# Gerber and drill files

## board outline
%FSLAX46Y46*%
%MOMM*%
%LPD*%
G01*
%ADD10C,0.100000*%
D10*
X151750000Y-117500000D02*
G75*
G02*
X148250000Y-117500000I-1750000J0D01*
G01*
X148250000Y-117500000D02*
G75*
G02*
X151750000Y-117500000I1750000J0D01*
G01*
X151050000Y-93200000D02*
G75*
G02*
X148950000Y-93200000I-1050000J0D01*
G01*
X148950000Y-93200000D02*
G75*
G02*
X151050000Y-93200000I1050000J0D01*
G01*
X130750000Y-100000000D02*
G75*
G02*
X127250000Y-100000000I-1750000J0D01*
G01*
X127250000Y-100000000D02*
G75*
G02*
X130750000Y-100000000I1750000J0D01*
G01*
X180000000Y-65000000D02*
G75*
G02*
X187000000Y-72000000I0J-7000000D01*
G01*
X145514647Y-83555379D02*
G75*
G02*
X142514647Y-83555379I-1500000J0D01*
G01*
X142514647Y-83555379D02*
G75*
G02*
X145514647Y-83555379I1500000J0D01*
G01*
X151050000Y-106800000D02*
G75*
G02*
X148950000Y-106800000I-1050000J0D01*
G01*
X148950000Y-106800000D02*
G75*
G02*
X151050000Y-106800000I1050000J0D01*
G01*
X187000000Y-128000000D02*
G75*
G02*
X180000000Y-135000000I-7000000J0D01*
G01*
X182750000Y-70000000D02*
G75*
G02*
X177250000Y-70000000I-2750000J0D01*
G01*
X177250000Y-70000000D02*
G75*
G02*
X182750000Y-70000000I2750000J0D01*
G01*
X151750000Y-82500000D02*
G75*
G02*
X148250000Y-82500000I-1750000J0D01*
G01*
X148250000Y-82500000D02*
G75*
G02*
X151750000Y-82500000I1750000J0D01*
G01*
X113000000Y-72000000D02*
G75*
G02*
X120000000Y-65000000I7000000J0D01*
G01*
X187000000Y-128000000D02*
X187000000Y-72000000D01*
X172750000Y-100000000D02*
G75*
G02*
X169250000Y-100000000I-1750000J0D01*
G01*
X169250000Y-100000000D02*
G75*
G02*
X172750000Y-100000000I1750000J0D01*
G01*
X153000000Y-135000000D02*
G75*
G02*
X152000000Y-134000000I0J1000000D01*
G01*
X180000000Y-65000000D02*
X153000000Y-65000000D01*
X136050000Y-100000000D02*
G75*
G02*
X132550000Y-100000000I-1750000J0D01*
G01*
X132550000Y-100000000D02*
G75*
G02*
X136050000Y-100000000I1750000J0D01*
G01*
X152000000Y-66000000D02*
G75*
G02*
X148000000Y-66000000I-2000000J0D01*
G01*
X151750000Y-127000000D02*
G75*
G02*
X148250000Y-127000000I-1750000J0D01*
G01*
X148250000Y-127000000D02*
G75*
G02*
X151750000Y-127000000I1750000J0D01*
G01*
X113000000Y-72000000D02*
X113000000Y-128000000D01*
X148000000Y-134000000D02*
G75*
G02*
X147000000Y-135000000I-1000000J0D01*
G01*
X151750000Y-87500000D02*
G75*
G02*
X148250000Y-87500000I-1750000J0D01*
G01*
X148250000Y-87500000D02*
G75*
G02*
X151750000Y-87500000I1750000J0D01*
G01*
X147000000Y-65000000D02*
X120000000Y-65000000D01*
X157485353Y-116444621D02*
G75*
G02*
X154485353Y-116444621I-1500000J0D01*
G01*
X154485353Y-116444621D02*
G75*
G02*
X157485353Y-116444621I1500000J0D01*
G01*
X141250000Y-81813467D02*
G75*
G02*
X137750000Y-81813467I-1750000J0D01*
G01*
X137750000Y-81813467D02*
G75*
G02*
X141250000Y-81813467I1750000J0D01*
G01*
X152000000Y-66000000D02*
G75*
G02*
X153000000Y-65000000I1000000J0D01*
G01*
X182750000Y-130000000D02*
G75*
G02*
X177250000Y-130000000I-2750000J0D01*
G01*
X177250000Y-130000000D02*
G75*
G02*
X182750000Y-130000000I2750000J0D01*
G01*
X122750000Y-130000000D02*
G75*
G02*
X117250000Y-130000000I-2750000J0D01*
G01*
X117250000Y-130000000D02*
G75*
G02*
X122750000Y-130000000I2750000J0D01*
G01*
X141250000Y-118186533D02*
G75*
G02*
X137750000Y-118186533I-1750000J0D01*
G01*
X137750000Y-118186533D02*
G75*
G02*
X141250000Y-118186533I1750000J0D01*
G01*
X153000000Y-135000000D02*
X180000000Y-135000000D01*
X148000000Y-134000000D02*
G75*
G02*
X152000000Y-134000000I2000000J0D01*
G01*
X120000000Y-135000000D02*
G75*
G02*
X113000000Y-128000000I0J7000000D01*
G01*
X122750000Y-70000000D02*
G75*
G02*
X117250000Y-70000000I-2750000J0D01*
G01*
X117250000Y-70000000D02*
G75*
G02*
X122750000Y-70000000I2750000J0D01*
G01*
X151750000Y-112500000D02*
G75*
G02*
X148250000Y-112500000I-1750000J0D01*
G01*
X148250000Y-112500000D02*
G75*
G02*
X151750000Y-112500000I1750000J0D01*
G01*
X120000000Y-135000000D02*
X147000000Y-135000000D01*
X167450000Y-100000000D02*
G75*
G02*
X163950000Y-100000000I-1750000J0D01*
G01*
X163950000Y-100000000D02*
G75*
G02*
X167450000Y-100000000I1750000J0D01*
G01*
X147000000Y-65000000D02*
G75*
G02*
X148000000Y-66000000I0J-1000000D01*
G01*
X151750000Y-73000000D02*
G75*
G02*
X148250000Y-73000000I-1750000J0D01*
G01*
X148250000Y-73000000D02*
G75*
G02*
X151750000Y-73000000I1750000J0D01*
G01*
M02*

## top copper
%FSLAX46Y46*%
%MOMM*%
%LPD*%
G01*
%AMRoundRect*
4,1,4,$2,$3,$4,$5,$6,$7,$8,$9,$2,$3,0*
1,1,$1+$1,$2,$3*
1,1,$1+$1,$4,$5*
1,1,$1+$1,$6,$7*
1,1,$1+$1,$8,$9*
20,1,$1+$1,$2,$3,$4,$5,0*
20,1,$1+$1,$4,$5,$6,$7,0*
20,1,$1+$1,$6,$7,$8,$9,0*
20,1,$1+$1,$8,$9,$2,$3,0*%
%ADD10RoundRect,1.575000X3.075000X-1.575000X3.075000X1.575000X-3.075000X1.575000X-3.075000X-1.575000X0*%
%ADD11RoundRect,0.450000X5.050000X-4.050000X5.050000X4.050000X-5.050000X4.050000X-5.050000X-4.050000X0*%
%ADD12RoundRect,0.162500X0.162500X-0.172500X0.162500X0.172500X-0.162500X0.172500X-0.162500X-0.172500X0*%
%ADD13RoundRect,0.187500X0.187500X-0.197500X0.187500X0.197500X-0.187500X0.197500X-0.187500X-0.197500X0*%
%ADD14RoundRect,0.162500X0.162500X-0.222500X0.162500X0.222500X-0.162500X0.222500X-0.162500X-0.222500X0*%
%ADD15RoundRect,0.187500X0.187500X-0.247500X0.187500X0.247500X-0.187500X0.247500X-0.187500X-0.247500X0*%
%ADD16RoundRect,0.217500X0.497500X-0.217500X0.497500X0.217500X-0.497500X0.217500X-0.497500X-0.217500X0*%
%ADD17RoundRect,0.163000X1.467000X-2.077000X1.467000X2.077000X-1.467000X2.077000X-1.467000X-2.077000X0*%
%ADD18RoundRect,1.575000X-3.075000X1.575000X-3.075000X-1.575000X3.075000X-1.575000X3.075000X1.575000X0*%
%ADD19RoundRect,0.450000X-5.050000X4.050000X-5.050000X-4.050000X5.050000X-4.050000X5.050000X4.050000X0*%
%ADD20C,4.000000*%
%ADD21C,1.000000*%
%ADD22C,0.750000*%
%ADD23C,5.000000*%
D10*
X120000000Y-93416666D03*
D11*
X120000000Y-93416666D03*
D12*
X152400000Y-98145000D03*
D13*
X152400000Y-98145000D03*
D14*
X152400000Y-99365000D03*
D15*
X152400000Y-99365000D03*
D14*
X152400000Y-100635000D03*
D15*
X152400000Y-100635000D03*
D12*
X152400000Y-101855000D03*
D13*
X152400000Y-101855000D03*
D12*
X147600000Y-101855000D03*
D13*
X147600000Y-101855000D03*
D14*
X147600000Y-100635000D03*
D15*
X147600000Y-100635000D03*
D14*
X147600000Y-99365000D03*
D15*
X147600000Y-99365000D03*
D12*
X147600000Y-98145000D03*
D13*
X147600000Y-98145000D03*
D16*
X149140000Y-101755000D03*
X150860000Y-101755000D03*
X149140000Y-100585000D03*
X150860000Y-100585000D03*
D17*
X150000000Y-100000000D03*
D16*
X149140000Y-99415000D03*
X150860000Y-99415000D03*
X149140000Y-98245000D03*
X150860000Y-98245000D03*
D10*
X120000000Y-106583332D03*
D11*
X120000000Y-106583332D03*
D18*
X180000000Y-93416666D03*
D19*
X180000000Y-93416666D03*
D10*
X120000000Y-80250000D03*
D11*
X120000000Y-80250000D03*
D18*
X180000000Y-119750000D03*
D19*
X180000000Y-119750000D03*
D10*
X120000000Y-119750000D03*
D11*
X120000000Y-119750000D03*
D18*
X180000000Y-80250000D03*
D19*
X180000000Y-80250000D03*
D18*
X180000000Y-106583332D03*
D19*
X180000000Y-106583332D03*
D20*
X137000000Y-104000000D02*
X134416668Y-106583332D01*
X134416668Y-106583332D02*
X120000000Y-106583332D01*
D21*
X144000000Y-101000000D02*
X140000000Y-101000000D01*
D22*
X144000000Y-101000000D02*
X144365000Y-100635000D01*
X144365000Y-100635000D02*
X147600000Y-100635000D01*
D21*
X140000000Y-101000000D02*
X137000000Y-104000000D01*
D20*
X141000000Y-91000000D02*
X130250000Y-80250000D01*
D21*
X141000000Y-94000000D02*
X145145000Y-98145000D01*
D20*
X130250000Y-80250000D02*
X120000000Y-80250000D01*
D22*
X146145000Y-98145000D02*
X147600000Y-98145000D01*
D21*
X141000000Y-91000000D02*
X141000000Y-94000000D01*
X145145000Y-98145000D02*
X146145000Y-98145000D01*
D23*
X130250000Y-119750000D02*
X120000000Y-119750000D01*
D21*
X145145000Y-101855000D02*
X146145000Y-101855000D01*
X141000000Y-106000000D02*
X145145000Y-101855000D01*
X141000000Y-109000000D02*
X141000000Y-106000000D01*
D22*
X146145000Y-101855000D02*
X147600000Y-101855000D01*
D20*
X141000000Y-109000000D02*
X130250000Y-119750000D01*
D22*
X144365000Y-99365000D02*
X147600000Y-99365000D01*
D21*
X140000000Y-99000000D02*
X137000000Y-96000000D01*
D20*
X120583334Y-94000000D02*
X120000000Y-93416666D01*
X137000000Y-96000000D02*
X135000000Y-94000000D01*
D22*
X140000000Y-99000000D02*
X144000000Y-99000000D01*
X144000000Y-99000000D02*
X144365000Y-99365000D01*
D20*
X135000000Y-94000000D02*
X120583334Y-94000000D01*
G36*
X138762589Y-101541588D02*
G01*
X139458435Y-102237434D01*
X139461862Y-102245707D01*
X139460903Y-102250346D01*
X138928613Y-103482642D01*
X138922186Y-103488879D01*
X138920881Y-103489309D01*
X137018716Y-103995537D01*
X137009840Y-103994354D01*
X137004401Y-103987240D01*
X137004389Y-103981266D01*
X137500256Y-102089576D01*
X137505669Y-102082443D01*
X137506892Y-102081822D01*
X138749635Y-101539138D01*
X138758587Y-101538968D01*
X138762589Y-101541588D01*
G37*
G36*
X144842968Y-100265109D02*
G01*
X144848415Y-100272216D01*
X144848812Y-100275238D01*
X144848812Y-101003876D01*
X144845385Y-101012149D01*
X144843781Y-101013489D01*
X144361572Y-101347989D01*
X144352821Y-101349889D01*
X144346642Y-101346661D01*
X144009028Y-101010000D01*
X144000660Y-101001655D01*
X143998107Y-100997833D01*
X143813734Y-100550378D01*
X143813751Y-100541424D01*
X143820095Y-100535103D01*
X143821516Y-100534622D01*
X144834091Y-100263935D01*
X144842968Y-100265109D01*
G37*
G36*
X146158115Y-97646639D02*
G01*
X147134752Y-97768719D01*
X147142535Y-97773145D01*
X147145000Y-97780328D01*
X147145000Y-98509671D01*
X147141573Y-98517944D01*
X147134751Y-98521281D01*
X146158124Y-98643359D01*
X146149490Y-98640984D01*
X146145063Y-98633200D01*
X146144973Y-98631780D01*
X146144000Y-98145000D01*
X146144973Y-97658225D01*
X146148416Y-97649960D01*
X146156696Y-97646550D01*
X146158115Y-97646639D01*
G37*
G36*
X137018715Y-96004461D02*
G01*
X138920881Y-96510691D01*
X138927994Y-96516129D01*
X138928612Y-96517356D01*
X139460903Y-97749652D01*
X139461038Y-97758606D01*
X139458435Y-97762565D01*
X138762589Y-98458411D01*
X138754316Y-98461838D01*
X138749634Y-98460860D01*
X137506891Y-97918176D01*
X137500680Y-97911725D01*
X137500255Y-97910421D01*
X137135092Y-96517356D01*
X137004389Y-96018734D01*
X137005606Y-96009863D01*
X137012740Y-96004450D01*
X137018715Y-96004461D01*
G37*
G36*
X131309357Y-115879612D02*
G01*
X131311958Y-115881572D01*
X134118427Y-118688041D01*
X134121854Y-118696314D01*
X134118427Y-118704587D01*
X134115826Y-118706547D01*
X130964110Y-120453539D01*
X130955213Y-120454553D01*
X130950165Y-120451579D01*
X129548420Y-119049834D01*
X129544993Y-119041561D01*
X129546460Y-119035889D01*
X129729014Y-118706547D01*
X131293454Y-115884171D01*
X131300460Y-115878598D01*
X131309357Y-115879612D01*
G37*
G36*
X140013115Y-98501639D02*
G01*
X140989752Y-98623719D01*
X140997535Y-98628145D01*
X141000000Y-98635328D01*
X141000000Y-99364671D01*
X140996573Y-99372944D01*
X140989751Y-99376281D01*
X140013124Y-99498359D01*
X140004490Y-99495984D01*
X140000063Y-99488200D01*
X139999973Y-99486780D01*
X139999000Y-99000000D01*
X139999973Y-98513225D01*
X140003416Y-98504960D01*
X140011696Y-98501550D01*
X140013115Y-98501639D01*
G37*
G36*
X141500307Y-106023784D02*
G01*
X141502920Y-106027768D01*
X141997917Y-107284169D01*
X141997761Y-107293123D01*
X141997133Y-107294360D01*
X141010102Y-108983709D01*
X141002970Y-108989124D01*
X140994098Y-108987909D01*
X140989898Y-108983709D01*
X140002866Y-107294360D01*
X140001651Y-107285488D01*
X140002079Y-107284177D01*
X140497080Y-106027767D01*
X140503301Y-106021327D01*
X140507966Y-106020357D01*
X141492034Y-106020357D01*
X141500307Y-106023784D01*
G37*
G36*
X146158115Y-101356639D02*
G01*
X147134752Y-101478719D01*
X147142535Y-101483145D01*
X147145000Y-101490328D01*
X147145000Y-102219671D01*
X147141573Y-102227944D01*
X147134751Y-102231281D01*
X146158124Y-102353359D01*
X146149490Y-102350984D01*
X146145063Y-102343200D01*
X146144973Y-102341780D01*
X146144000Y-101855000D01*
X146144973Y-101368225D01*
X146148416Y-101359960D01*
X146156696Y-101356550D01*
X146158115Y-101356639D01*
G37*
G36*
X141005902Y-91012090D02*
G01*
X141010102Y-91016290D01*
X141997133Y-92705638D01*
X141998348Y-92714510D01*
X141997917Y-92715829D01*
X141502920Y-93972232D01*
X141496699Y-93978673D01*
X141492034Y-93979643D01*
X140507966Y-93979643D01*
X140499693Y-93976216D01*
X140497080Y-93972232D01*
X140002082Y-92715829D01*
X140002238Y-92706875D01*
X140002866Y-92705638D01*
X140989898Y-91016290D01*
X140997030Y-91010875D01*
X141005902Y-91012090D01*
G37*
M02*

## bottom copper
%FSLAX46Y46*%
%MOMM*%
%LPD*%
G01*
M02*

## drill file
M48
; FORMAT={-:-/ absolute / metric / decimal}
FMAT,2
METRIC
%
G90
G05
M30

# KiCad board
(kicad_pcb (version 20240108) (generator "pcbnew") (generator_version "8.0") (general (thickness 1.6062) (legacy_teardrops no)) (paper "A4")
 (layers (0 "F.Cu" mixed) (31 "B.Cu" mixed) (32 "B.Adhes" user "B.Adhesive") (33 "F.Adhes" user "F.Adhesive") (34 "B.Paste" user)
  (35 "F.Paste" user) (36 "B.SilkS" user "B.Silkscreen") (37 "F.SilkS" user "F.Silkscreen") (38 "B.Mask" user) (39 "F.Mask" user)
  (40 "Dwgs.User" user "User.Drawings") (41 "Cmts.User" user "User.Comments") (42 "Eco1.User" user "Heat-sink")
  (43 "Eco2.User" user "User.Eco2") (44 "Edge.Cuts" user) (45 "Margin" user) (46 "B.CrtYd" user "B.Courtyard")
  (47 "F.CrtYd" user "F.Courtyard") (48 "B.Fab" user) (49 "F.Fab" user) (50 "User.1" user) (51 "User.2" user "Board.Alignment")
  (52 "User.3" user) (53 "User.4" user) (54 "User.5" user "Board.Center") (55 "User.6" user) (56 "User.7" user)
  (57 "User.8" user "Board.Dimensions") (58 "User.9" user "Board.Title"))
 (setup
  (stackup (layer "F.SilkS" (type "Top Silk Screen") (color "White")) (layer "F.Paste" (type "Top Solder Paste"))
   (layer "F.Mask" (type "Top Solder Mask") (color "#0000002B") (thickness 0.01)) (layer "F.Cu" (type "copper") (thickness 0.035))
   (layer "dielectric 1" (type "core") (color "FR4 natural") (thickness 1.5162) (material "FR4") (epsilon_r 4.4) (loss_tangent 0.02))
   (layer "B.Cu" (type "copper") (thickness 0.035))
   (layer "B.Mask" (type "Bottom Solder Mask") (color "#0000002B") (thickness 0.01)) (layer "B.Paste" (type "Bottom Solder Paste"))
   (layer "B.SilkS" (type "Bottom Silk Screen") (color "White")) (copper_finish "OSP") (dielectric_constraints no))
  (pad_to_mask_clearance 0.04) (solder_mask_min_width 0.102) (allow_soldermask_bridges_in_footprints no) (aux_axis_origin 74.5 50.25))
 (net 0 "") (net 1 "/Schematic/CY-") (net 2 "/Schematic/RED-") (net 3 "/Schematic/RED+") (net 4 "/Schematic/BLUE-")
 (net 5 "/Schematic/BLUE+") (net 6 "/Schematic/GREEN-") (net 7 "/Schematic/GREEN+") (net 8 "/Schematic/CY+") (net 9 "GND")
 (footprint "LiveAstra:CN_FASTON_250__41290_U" (layer "F.Cu") (at 120 93.416666 90)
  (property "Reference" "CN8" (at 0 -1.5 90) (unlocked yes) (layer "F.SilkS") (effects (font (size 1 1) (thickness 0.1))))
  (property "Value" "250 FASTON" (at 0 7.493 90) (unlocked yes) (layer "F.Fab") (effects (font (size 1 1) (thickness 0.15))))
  (pad "1" smd roundrect (at 0 0 90) (size 6.3 9.3) (layers "F.Cu" "F.Paste") (roundrect_rratio 0.25) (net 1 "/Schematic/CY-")
   (thermal_bridge_angle 45)
   (teardrops (best_length_ratio 0.5) (max_length 1) (best_width_ratio 1) (max_width 2) (curve_points 0) (filter_ratio 0.9) (enabled yes)
    (allow_two_segments yes) (prefer_zone_connections yes)))
  (pad "1" smd roundrect (at 0 0 90) (size 9 11) (layers "F.Cu" "F.Mask") (roundrect_rratio 0.05) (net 1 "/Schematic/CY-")
   (thermal_bridge_angle 45)
   (teardrops (best_length_ratio 0.5) (max_length 1) (best_width_ratio 1) (max_width 2) (curve_points 0) (filter_ratio 0.9) (enabled yes)
    (allow_two_segments yes) (prefer_zone_connections yes))))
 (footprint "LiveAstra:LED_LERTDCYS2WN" (layer "F.Cu") (at 150 100 90)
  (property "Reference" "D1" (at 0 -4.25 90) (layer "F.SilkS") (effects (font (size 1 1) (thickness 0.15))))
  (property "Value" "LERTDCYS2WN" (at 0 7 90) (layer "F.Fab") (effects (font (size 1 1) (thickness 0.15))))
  (pad "1" smd roundrect (at 1.855 2.4 90) (size 0.67 0.65) (layers "F.Cu" "F.Paste") (roundrect_rratio 0.25) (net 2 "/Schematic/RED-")
   (thermal_bridge_angle 45)
   (teardrops (best_length_ratio 0.5) (max_length 1) (best_width_ratio 1) (max_width 2) (curve_points 0) (filter_ratio 0.9) (enabled yes)
    (allow_two_segments yes) (prefer_zone_connections yes)))
  (pad "1" smd roundrect (at 1.855 2.4 90) (size 0.77 0.75) (layers "F.Cu" "F.Mask") (roundrect_rratio 0.25) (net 2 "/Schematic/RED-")
   (thermal_bridge_angle 45)
   (teardrops (best_length_ratio 0.5) (max_length 1) (best_width_ratio 1) (max_width 2) (curve_points 0) (filter_ratio 0.9) (enabled yes)
    (allow_two_segments yes) (prefer_zone_connections yes)))
  (pad "2" smd roundrect (at 0.635 2.4 90) (size 0.77 0.65) (layers "F.Cu" "F.Paste") (roundrect_rratio 0.25) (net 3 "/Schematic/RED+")
   (thermal_bridge_angle 45)
   (teardrops (best_length_ratio 0.5) (max_length 1) (best_width_ratio 1) (max_width 2) (curve_points 0) (filter_ratio 0.9) (enabled yes)
    (allow_two_segments yes) (prefer_zone_connections yes)))
  (pad "2" smd roundrect (at 0.635 2.4 90) (size 0.87 0.75) (layers "F.Cu" "F.Mask") (roundrect_rratio 0.25) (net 3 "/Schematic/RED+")
   (thermal_bridge_angle 45)
   (teardrops (best_length_ratio 0.5) (max_length 1) (best_width_ratio 1) (max_width 2) (curve_points 0) (filter_ratio 0.9) (enabled yes)
    (allow_two_segments yes) (prefer_zone_connections yes)))
  (pad "3" smd roundrect (at -0.635 2.4 90) (size 0.77 0.65) (layers "F.Cu" "F.Paste") (roundrect_rratio 0.25) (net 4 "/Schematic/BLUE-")
   (thermal_bridge_angle 45)
   (teardrops (best_length_ratio 0.5) (max_length 1) (best_width_ratio 1) (max_width 2) (curve_points 0) (filter_ratio 0.9) (enabled yes)
    (allow_two_segments yes) (prefer_zone_connections yes)))
  (pad "3" smd roundrect (at -0.635 2.4 90) (size 0.87 0.75) (layers "F.Cu" "F.Mask") (roundrect_rratio 0.25) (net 4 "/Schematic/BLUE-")
   (thermal_bridge_angle 45)
   (teardrops (best_length_ratio 0.5) (max_length 1) (best_width_ratio 1) (max_width 2) (curve_points 0) (filter_ratio 0.9) (enabled yes)
    (allow_two_segments yes) (prefer_zone_connections yes)))
  (pad "4" smd roundrect (at -1.855 2.4 90) (size 0.67 0.65) (layers "F.Cu" "F.Paste") (roundrect_rratio 0.25) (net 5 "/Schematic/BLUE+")
   (thermal_bridge_angle 45)
   (teardrops (best_length_ratio 0.5) (max_length 1) (best_width_ratio 1) (max_width 2) (curve_points 0) (filter_ratio 0.9) (enabled yes)
    (allow_two_segments yes) (prefer_zone_connections yes)))
  (pad "4" smd roundrect (at -1.855 2.4 90) (size 0.77 0.75) (layers "F.Cu" "F.Mask") (roundrect_rratio 0.25) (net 5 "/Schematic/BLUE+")
   (thermal_bridge_angle 45)
   (teardrops (best_length_ratio 0.5) (max_length 1) (best_width_ratio 1) (max_width 2) (curve_points 0) (filter_ratio 0.9) (enabled yes)
    (allow_two_segments yes) (prefer_zone_connections yes)))
  (pad "5" smd roundrect (at -1.855 -2.4 90) (size 0.67 0.65) (layers "F.Cu" "F.Paste") (roundrect_rratio 0.25) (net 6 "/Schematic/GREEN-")
   (thermal_bridge_angle 45)
   (teardrops (best_length_ratio 0.5) (max_length 1) (best_width_ratio 1) (max_width 2) (curve_points 0) (filter_ratio 0.9) (enabled yes)
    (allow_two_segments yes) (prefer_zone_connections yes)))
  (pad "5" smd roundrect (at -1.855 -2.4 90) (size 0.77 0.75) (layers "F.Cu" "F.Mask") (roundrect_rratio 0.25) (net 6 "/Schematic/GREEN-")
   (thermal_bridge_angle 45)
   (teardrops (best_length_ratio 0.5) (max_length 1) (best_width_ratio 1) (max_width 2) (curve_points 0) (filter_ratio 0.9) (enabled yes)
    (allow_two_segments yes) (prefer_zone_connections yes)))
  (pad "6" smd roundrect (at -0.635 -2.4 90) (size 0.77 0.65) (layers "F.Cu" "F.Paste") (roundrect_rratio 0.25) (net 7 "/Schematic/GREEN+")
   (thermal_bridge_angle 45)
   (teardrops (best_length_ratio 0.5) (max_length 1) (best_width_ratio 1) (max_width 2) (curve_points 0) (filter_ratio 0.9) (enabled yes)
    (allow_two_segments yes) (prefer_zone_connections yes)))
  (pad "6" smd roundrect (at -0.635 -2.4 90) (size 0.87 0.75) (layers "F.Cu" "F.Mask") (roundrect_rratio 0.25) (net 7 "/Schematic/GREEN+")
   (thermal_bridge_angle 45)
   (teardrops (best_length_ratio 0.5) (max_length 1) (best_width_ratio 1) (max_width 2) (curve_points 0) (filter_ratio 0.9) (enabled yes)
    (allow_two_segments yes) (prefer_zone_connections yes)))
  (pad "7" smd roundrect (at 0.635 -2.4 90) (size 0.77 0.65) (layers "F.Cu" "F.Paste") (roundrect_rratio 0.25) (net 1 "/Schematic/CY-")
   (thermal_bridge_angle 45)
   (teardrops (best_length_ratio 0.5) (max_length 1) (best_width_ratio 1) (max_width 2) (curve_points 0) (filter_ratio 0.9) (enabled yes)
    (allow_two_segments yes) (prefer_zone_connections yes)))
  (pad "7" smd roundrect (at 0.635 -2.4 90) (size 0.87 0.75) (layers "F.Cu" "F.Mask") (roundrect_rratio 0.25) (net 1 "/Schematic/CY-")
   (thermal_bridge_angle 45)
   (teardrops (best_length_ratio 0.5) (max_length 1) (best_width_ratio 1) (max_width 2) (curve_points 0) (filter_ratio 0.9) (enabled yes)
    (allow_two_segments yes) (prefer_zone_connections yes)))
  (pad "8" smd roundrect (at 1.855 -2.4 90) (size 0.67 0.65) (layers "F.Cu" "F.Paste") (roundrect_rratio 0.25) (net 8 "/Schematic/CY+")
   (thermal_bridge_angle 45)
   (teardrops (best_length_ratio 0.5) (max_length 1) (best_width_ratio 1) (max_width 2) (curve_points 0) (filter_ratio 0.9) (enabled yes)
    (allow_two_segments yes) (prefer_zone_connections yes)))
  (pad "8" smd roundrect (at 1.855 -2.4 90) (size 0.77 0.75) (layers "F.Cu" "F.Mask") (roundrect_rratio 0.25) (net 8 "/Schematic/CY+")
   (thermal_bridge_angle 45)
   (teardrops (best_length_ratio 0.5) (max_length 1) (best_width_ratio 1) (max_width 2) (curve_points 0) (filter_ratio 0.9) (enabled yes)
    (allow_two_segments yes) (prefer_zone_connections yes)))
  (pad "9" smd roundrect (at -1.755 -0.86 90) (size 0.87 1.43) (layers "F.Cu" "F.Paste") (roundrect_rratio 0.25) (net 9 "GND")
   (thermal_bridge_angle 45)
   (teardrops (best_length_ratio 0.5) (max_length 1) (best_width_ratio 1) (max_width 2) (curve_points 0) (filter_ratio 0.9) (enabled yes)
    (allow_two_segments yes) (prefer_zone_connections yes)))
  (pad "9" smd roundrect (at -1.755 0.86 90) (size 0.87 1.43) (layers "F.Cu" "F.Paste") (roundrect_rratio 0.25) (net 9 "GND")
   (thermal_bridge_angle 45)
   (teardrops (best_length_ratio 0.5) (max_length 1) (best_width_ratio 1) (max_width 2) (curve_points 0) (filter_ratio 0.9) (enabled yes)
    (allow_two_segments yes) (prefer_zone_connections yes)))
  (pad "9" smd roundrect (at -0.585 -0.86 90) (size 0.87 1.43) (layers "F.Cu" "F.Paste") (roundrect_rratio 0.25) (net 9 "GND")
   (thermal_bridge_angle 45)
   (teardrops (best_length_ratio 0.5) (max_length 1) (best_width_ratio 1) (max_width 2) (curve_points 0) (filter_ratio 0.9) (enabled yes)
    (allow_two_segments yes) (prefer_zone_connections yes)))
  (pad "9" smd roundrect (at -0.585 0.86 90) (size 0.87 1.43) (layers "F.Cu" "F.Paste") (roundrect_rratio 0.25) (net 9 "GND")
   (thermal_bridge_angle 45)
   (teardrops (best_length_ratio 0.5) (max_length 1) (best_width_ratio 1) (max_width 2) (curve_points 0) (filter_ratio 0.9) (enabled yes)
    (allow_two_segments yes) (prefer_zone_connections yes)))
  (pad "9" smd roundrect (at 0 0 90) (size 4.48 3.26) (layers "F.Cu" "F.Mask") (roundrect_rratio 0.05) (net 9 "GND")
   (thermal_bridge_angle 45)
   (teardrops (best_length_ratio 0.5) (max_length 1) (best_width_ratio 1) (max_width 2) (curve_points 0) (filter_ratio 0.9) (enabled yes)
    (allow_two_segments yes) (prefer_zone_connections yes)))
  (pad "9" smd roundrect (at 0.585 -0.86 90) (size 0.87 1.43) (layers "F.Cu" "F.Paste") (roundrect_rratio 0.25) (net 9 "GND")
   (thermal_bridge_angle 45)
   (teardrops (best_length_ratio 0.5) (max_length 1) (best_width_ratio 1) (max_width 2) (curve_points 0) (filter_ratio 0.9) (enabled yes)
    (allow_two_segments yes) (prefer_zone_connections yes)))
  (pad "9" smd roundrect (at 0.585 0.86 90) (size 0.87 1.43) (layers "F.Cu" "F.Paste") (roundrect_rratio 0.25) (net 9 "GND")
   (thermal_bridge_angle 45)
   (teardrops (best_length_ratio 0.5) (max_length 1) (best_width_ratio 1) (max_width 2) (curve_points 0) (filter_ratio 0.9) (enabled yes)
    (allow_two_segments yes) (prefer_zone_connections yes)))
  (pad "9" smd roundrect (at 1.755 -0.86 90) (size 0.87 1.43) (layers "F.Cu" "F.Paste") (roundrect_rratio 0.25) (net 9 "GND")
   (thermal_bridge_angle 45)
   (teardrops (best_length_ratio 0.5) (max_length 1) (best_width_ratio 1) (max_width 2) (curve_points 0) (filter_ratio 0.9) (enabled yes)
    (allow_two_segments yes) (prefer_zone_connections yes)))
  (pad "9" smd roundrect (at 1.755 0.86 90) (size 0.87 1.43) (layers "F.Cu" "F.Paste") (roundrect_rratio 0.25) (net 9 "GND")
   (thermal_bridge_angle 45)
   (teardrops (best_length_ratio 0.5) (max_length 1) (best_width_ratio 1) (max_width 2) (curve_points 0) (filter_ratio 0.9) (enabled yes)
    (allow_two_segments yes) (prefer_zone_connections yes))))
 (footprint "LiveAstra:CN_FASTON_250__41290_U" (layer "F.Cu") (at 120 106.583332 90)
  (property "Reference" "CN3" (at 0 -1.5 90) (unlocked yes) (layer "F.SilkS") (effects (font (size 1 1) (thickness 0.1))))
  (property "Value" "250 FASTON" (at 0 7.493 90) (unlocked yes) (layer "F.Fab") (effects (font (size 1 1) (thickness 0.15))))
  (pad "1" smd roundrect (at 0 0 90) (size 6.3 9.3) (layers "F.Cu" "F.Paste") (roundrect_rratio 0.25) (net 7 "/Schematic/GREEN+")
   (thermal_bridge_angle 45)
   (teardrops (best_length_ratio 0.5) (max_length 1) (best_width_ratio 1) (max_width 2) (curve_points 0) (filter_ratio 0.9) (enabled yes)
    (allow_two_segments yes) (prefer_zone_connections yes)))
  (pad "1" smd roundrect (at 0 0 90) (size 9 11) (layers "F.Cu" "F.Mask") (roundrect_rratio 0.05) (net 7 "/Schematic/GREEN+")
   (thermal_bridge_angle 45)
   (teardrops (best_length_ratio 0.5) (max_length 1) (best_width_ratio 1) (max_width 2) (curve_points 0) (filter_ratio 0.9) (enabled yes)
    (allow_two_segments yes) (prefer_zone_connections yes))))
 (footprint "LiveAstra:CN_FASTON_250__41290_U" (layer "F.Cu") (at 180 93.416666 -90)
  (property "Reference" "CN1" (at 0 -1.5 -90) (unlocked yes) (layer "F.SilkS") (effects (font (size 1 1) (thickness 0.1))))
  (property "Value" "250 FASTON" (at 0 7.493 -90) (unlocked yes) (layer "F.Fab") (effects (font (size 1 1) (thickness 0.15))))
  (pad "1" smd roundrect (at 0 0 270) (size 6.3 9.3) (layers "F.Cu" "F.Paste") (roundrect_rratio 0.25) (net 3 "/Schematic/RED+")
   (thermal_bridge_angle 45)
   (teardrops (best_length_ratio 0.5) (max_length 1) (best_width_ratio 1) (max_width 2) (curve_points 0) (filter_ratio 0.9) (enabled yes)
    (allow_two_segments yes) (prefer_zone_connections yes)))
  (pad "1" smd roundrect (at 0 0 270) (size 9 11) (layers "F.Cu" "F.Mask") (roundrect_rratio 0.05) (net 3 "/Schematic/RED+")
   (thermal_bridge_angle 45)
   (teardrops (best_length_ratio 0.5) (max_length 1) (best_width_ratio 1) (max_width 2) (curve_points 0) (filter_ratio 0.9) (enabled yes)
    (allow_two_segments yes) (prefer_zone_connections yes))))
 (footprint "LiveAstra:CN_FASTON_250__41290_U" (layer "F.Cu") (at 120 80.25 90)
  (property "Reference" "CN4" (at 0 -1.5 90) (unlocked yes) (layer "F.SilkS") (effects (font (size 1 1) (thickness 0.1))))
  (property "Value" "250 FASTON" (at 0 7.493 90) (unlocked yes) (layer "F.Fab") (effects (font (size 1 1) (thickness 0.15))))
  (pad "1" smd roundrect (at 0 0 90) (size 6.3 9.3) (layers "F.Cu" "F.Paste") (roundrect_rratio 0.25) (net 8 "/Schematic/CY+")
   (thermal_bridge_angle 45)
   (teardrops (best_length_ratio 0.5) (max_length 1) (best_width_ratio 1) (max_width 2) (curve_points 0) (filter_ratio 0.9) (enabled yes)
    (allow_two_segments yes) (prefer_zone_connections yes)))
  (pad "1" smd roundrect (at 0 0 90) (size 9 11) (layers "F.Cu" "F.Mask") (roundrect_rratio 0.05) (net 8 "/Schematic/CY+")
   (thermal_bridge_angle 45)
   (teardrops (best_length_ratio 0.5) (max_length 1) (best_width_ratio 1) (max_width 2) (curve_points 0) (filter_ratio 0.9) (enabled yes)
    (allow_two_segments yes) (prefer_zone_connections yes))))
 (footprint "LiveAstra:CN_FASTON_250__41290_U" (layer "F.Cu") (at 180 119.75 -90)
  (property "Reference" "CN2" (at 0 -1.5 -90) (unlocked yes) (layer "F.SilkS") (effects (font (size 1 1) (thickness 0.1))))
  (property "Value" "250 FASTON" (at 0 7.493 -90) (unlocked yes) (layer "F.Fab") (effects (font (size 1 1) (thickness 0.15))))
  (pad "1" smd roundrect (at 0 0 270) (size 6.3 9.3) (layers "F.Cu" "F.Paste") (roundrect_rratio 0.25) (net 5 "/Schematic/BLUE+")
   (thermal_bridge_angle 45)
   (teardrops (best_length_ratio 0.5) (max_length 1) (best_width_ratio 1) (max_width 2) (curve_points 0) (filter_ratio 0.9) (enabled yes)
    (allow_two_segments yes) (prefer_zone_connections yes)))
  (pad "1" smd roundrect (at 0 0 270) (size 9 11) (layers "F.Cu" "F.Mask") (roundrect_rratio 0.05) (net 5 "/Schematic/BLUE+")
   (thermal_bridge_angle 45)
   (teardrops (best_length_ratio 0.5) (max_length 1) (best_width_ratio 1) (max_width 2) (curve_points 0) (filter_ratio 0.9) (enabled yes)
    (allow_two_segments yes) (prefer_zone_connections yes))))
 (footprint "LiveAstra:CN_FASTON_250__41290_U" (layer "F.Cu") (at 120 119.75 90)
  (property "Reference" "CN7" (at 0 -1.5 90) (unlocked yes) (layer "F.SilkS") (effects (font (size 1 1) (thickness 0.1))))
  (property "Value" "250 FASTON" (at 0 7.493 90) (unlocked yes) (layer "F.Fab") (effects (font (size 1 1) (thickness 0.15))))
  (pad "1" smd roundrect (at 0 0 90) (size 6.3 9.3) (layers "F.Cu" "F.Paste") (roundrect_rratio 0.25) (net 6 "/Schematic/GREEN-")
   (thermal_bridge_angle 45)
   (teardrops (best_length_ratio 0.5) (max_length 1) (best_width_ratio 1) (max_width 2) (curve_points 0) (filter_ratio 0.9) (enabled yes)
    (allow_two_segments yes) (prefer_zone_connections yes)))
  (pad "1" smd roundrect (at 0 0 90) (size 9 11) (layers "F.Cu" "F.Mask") (roundrect_rratio 0.05) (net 6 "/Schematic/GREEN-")
   (thermal_bridge_angle 45)
   (teardrops (best_length_ratio 0.5) (max_length 1) (best_width_ratio 1) (max_width 2) (curve_points 0) (filter_ratio 0.9) (enabled yes)
    (allow_two_segments yes) (prefer_zone_connections yes))))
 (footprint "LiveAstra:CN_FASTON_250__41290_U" (layer "F.Cu") (at 180 80.25 -90)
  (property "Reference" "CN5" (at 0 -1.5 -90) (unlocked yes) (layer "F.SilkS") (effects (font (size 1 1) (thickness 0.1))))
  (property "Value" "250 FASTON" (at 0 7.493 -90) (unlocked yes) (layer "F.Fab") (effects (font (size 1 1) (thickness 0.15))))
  (pad "1" smd roundrect (at 0 0 270) (size 6.3 9.3) (layers "F.Cu" "F.Paste") (roundrect_rratio 0.25) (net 2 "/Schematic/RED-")
   (thermal_bridge_angle 45)
   (teardrops (best_length_ratio 0.5) (max_length 1) (best_width_ratio 1) (max_width 2) (curve_points 0) (filter_ratio 0.9) (enabled yes)
    (allow_two_segments yes) (prefer_zone_connections yes)))
  (pad "1" smd roundrect (at 0 0 270) (size 9 11) (layers "F.Cu" "F.Mask") (roundrect_rratio 0.05) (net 2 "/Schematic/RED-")
   (thermal_bridge_angle 45)
   (teardrops (best_length_ratio 0.5) (max_length 1) (best_width_ratio 1) (max_width 2) (curve_points 0) (filter_ratio 0.9) (enabled yes)
    (allow_two_segments yes) (prefer_zone_connections yes))))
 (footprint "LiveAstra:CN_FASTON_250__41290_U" (layer "F.Cu") (at 180 106.583332 -90)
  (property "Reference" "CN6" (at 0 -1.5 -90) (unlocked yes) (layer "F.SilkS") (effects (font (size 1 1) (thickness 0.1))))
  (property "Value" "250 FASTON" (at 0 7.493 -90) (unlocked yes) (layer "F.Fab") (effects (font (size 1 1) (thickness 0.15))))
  (pad "1" smd roundrect (at 0 0 270) (size 6.3 9.3) (layers "F.Cu" "F.Paste") (roundrect_rratio 0.25) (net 4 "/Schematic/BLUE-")
   (thermal_bridge_angle 45)
   (teardrops (best_length_ratio 0.5) (max_length 1) (best_width_ratio 1) (max_width 2) (curve_points 0) (filter_ratio 0.9) (enabled yes)
    (allow_two_segments yes) (prefer_zone_connections yes)))
  (pad "1" smd roundrect (at 0 0 270) (size 9 11) (layers "F.Cu" "F.Mask") (roundrect_rratio 0.05) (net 4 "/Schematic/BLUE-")
   (thermal_bridge_angle 45)
   (teardrops (best_length_ratio 0.5) (max_length 1) (best_width_ratio 1) (max_width 2) (curve_points 0) (filter_ratio 0.9) (enabled yes)
    (allow_two_segments yes) (prefer_zone_connections yes))))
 (gr_circle (center 150 117.5) (end 150 115.75) (stroke (width 0.1) (type default)) (fill none) (layer "Edge.Cuts"))
 (gr_circle (center 150 93.2) (end 150 92.15) (stroke (width 0.1) (type default)) (fill none) (layer "Edge.Cuts"))
 (gr_circle (center 129 100) (end 129 98.25) (stroke (width 0.1) (type default)) (fill none) (layer "Edge.Cuts"))
 (gr_arc (start 180 65) (mid 184.949747 67.050252) (end 187 72) (stroke (width 0.1) (type default)) (layer "Edge.Cuts"))
 (gr_circle (center 144.014647 83.555379) (end 144.014647 82.055379) (stroke (width 0.1) (type default)) (fill none) (layer "Edge.Cuts"))
 (gr_circle (center 150 106.8) (end 150 105.75) (stroke (width 0.1) (type default)) (fill none) (layer "Edge.Cuts"))
 (gr_arc (start 187 128) (mid 184.949745 132.94975) (end 180 135) (stroke (width 0.1) (type default)) (layer "Edge.Cuts"))
 (gr_circle (center 180 70) (end 182.75 70) (stroke (width 0.1) (type default)) (fill none) (layer "Edge.Cuts"))
 (gr_circle (center 150 82.5) (end 150 80.75) (stroke (width 0.1) (type default)) (fill none) (layer "Edge.Cuts"))
 (gr_arc (start 113 72) (mid 115.050266 67.050239) (end 120 65) (stroke (width 0.1) (type default)) (layer "Edge.Cuts"))
 (gr_line (start 187 128) (end 187 72) (stroke (width 0.1) (type default)) (layer "Edge.Cuts"))
 (gr_circle (center 171 100) (end 171 98.25) (stroke (width 0.1) (type default)) (fill none) (layer "Edge.Cuts"))
 (gr_arc (start 153 135) (mid 152.292893 134.707107) (end 152 134) (stroke (width 0.1) (type default)) (layer "Edge.Cuts"))
 (gr_line (start 180 65) (end 153 65) (stroke (width 0.1) (type default)) (layer "Edge.Cuts"))
 (gr_circle (center 134.3 100) (end 134.3 98.25) (stroke (width 0.1) (type default)) (fill none) (layer "Edge.Cuts"))
 (gr_arc (start 152 66) (mid 150 68) (end 148 66) (stroke (width 0.1) (type default)) (layer "Edge.Cuts"))
 (gr_circle (center 150 127) (end 150 125.25) (stroke (width 0.1) (type default)) (fill none) (layer "Edge.Cuts"))
 (gr_line (start 113 72) (end 113 128) (stroke (width 0.1) (type default)) (layer "Edge.Cuts"))
 (gr_arc (start 148 134) (mid 147.707107 134.707107) (end 147 135) (stroke (width 0.1) (type default)) (layer "Edge.Cuts"))
 (gr_circle (center 150 87.5) (end 150 85.75) (stroke (width 0.1) (type default)) (fill none) (layer "Edge.Cuts"))
 (gr_line (start 147 65) (end 120 65) (stroke (width 0.1) (type default)) (layer "Edge.Cuts"))
 (gr_circle (center 155.985353 116.444621) (end 155.985353 114.944621) (stroke (width 0.1) (type default)) (fill none) (layer "Edge.Cuts"))
 (gr_circle (center 139.5 81.813467) (end 139.5 80.063467) (stroke (width 0.1) (type default)) (fill none) (layer "Edge.Cuts"))
 (gr_arc (start 152 66) (mid 152.292893 65.292893) (end 153 65) (stroke (width 0.1) (type default)) (layer "Edge.Cuts"))
 (gr_circle (center 180 130) (end 182.75 130) (stroke (width 0.1) (type default)) (fill none) (layer "Edge.Cuts"))
 (gr_circle (center 120 130) (end 122.75 130) (stroke (width 0.1) (type default)) (fill none) (layer "Edge.Cuts"))
 (gr_circle (center 139.5 118.186533) (end 139.5 116.436533) (stroke (width 0.1) (type default)) (fill none) (layer "Edge.Cuts"))
 (gr_line (start 153 135) (end 180 135) (stroke (width 0.1) (type default)) (layer "Edge.Cuts"))
 (gr_arc (start 148 134) (mid 150 132) (end 152 134) (stroke (width 0.1) (type default)) (layer "Edge.Cuts"))
 (gr_arc (start 120 135) (mid 115.050253 132.949747) (end 113 128) (stroke (width 0.1) (type default)) (layer "Edge.Cuts"))
 (gr_circle (center 120 70) (end 122.75 70) (stroke (width 0.1) (type default)) (fill none) (layer "Edge.Cuts"))
 (gr_circle (center 150 112.5) (end 150 110.75) (stroke (width 0.1) (type default)) (fill none) (layer "Edge.Cuts"))
 (gr_line (start 120 135) (end 147 135) (stroke (width 0.1) (type default)) (layer "Edge.Cuts"))
 (gr_circle (center 165.7 100) (end 165.7 98.25) (stroke (width 0.1) (type default)) (fill none) (layer "Edge.Cuts"))
 (gr_arc (start 147 65) (mid 147.707107 65.292893) (end 148 66) (stroke (width 0.1) (type default)) (layer "Edge.Cuts"))
 (gr_circle (center 150 73) (end 150 71.25) (stroke (width 0.1) (type default)) (fill none) (layer "Edge.Cuts"))
 (segment (start 137 104) (end 134.416668 106.583332) (width 4) (layer "F.Cu") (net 7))
 (segment (start 134.416668 106.583332) (end 120 106.583332) (width 4) (layer "F.Cu") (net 7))
 (segment (start 144 101) (end 140 101) (width 1) (layer "F.Cu") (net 7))
 (segment (start 144 101) (end 144.365 100.635) (width 0.75) (layer "F.Cu") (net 7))
 (segment (start 144.365 100.635) (end 147.6 100.635) (width 0.75) (layer "F.Cu") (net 7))
 (segment (start 140 101) (end 137 104) (width 1) (layer "F.Cu") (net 7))
 (segment (start 141 91) (end 130.25 80.25) (width 4) (layer "F.Cu") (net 8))
 (segment (start 141 94) (end 145.145 98.145) (width 1) (layer "F.Cu") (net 8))
 (segment (start 130.25 80.25) (end 120 80.25) (width 4) (layer "F.Cu") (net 8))
 (segment (start 146.145 98.145) (end 147.6 98.145) (width 0.75) (layer "F.Cu") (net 8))
 (segment (start 141 91) (end 141 94) (width 1) (layer "F.Cu") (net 8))
 (segment (start 145.145 98.145) (end 146.145 98.145) (width 1) (layer "F.Cu") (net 8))
 (segment (start 130.25 119.75) (end 120 119.75) (width 5) (layer "F.Cu") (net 6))
 (segment (start 145.145 101.855) (end 146.145 101.855) (width 1) (layer "F.Cu") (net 6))
 (segment (start 141 106) (end 145.145 101.855) (width 1) (layer "F.Cu") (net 6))
 (segment (start 141 109) (end 141 106) (width 1) (layer "F.Cu") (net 6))
 (segment (start 146.145 101.855) (end 147.6 101.855) (width 0.75) (layer "F.Cu") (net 6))
 (segment (start 141 109) (end 130.25 119.75) (width 4) (layer "F.Cu") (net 6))
 (segment (start 144.365 99.365) (end 147.6 99.365) (width 0.75) (layer "F.Cu") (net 1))
 (segment (start 140 99) (end 137 96) (width 1) (layer "F.Cu") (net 1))
 (segment (start 120.583334 94) (end 120 93.416666) (width 4) (layer "F.Cu") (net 1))
 (segment (start 137 96) (end 135 94) (width 4) (layer "F.Cu") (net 1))
 (segment (start 140 99) (end 144 99) (width 0.75) (layer "F.Cu") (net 1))
 (segment (start 144 99) (end 144.365 99.365) (width 0.75) (layer "F.Cu") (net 1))
 (segment (start 135 94) (end 120.583334 94) (width 4) (layer "F.Cu") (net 1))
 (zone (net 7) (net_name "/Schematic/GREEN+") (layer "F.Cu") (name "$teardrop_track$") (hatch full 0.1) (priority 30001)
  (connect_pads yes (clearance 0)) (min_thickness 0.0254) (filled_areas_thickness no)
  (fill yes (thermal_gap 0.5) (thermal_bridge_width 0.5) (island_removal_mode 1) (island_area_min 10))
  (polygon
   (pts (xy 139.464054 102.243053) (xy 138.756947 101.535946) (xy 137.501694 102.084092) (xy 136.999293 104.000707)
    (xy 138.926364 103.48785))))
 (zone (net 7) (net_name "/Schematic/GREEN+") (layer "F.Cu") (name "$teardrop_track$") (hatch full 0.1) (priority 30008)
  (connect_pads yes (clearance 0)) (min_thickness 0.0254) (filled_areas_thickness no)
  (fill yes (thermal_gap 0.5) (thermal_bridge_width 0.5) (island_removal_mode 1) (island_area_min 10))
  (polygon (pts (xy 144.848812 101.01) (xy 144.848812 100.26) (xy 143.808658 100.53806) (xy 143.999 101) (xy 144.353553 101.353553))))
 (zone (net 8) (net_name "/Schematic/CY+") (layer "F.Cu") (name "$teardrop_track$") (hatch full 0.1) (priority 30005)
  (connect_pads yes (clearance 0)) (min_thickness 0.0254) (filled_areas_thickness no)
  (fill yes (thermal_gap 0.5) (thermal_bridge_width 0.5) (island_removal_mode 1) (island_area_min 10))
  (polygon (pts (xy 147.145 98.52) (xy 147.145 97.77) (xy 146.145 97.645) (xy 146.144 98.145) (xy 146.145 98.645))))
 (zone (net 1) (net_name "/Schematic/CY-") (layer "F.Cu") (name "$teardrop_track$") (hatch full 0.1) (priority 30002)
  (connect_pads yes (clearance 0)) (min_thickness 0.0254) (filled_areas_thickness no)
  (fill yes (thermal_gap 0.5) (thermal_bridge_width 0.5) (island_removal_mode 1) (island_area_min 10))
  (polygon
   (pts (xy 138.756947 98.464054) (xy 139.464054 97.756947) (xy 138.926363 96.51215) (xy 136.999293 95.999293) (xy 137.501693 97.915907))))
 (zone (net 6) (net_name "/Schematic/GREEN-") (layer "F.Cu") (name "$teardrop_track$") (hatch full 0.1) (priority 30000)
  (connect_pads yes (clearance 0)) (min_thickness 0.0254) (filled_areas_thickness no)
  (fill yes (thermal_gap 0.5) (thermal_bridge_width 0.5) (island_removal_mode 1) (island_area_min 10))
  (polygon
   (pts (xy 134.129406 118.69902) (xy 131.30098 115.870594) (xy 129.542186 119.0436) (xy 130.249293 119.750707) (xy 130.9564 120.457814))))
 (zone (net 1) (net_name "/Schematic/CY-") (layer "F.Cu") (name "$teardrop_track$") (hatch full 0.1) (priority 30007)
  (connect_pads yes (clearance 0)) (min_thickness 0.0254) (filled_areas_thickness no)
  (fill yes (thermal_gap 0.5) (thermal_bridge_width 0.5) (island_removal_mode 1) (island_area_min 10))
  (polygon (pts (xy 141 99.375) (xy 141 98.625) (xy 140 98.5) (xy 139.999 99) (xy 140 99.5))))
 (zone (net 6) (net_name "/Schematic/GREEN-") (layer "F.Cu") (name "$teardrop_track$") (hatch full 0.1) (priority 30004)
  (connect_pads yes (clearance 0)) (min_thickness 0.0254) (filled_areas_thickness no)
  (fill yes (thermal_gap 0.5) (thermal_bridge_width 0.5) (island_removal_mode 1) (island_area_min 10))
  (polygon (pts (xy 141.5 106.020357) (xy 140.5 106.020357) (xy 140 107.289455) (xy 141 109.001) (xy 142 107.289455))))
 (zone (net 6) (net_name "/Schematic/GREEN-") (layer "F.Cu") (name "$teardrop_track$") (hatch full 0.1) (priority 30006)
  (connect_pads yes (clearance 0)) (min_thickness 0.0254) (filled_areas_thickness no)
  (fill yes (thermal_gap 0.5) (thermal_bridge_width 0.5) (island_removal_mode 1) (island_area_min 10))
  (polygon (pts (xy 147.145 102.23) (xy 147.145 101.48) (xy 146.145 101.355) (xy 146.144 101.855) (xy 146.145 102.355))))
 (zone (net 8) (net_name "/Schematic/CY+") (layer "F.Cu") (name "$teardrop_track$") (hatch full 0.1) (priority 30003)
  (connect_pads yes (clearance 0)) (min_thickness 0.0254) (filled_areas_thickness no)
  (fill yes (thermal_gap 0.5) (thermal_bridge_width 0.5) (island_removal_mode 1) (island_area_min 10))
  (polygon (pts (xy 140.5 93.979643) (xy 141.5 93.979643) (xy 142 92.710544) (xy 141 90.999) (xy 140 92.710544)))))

